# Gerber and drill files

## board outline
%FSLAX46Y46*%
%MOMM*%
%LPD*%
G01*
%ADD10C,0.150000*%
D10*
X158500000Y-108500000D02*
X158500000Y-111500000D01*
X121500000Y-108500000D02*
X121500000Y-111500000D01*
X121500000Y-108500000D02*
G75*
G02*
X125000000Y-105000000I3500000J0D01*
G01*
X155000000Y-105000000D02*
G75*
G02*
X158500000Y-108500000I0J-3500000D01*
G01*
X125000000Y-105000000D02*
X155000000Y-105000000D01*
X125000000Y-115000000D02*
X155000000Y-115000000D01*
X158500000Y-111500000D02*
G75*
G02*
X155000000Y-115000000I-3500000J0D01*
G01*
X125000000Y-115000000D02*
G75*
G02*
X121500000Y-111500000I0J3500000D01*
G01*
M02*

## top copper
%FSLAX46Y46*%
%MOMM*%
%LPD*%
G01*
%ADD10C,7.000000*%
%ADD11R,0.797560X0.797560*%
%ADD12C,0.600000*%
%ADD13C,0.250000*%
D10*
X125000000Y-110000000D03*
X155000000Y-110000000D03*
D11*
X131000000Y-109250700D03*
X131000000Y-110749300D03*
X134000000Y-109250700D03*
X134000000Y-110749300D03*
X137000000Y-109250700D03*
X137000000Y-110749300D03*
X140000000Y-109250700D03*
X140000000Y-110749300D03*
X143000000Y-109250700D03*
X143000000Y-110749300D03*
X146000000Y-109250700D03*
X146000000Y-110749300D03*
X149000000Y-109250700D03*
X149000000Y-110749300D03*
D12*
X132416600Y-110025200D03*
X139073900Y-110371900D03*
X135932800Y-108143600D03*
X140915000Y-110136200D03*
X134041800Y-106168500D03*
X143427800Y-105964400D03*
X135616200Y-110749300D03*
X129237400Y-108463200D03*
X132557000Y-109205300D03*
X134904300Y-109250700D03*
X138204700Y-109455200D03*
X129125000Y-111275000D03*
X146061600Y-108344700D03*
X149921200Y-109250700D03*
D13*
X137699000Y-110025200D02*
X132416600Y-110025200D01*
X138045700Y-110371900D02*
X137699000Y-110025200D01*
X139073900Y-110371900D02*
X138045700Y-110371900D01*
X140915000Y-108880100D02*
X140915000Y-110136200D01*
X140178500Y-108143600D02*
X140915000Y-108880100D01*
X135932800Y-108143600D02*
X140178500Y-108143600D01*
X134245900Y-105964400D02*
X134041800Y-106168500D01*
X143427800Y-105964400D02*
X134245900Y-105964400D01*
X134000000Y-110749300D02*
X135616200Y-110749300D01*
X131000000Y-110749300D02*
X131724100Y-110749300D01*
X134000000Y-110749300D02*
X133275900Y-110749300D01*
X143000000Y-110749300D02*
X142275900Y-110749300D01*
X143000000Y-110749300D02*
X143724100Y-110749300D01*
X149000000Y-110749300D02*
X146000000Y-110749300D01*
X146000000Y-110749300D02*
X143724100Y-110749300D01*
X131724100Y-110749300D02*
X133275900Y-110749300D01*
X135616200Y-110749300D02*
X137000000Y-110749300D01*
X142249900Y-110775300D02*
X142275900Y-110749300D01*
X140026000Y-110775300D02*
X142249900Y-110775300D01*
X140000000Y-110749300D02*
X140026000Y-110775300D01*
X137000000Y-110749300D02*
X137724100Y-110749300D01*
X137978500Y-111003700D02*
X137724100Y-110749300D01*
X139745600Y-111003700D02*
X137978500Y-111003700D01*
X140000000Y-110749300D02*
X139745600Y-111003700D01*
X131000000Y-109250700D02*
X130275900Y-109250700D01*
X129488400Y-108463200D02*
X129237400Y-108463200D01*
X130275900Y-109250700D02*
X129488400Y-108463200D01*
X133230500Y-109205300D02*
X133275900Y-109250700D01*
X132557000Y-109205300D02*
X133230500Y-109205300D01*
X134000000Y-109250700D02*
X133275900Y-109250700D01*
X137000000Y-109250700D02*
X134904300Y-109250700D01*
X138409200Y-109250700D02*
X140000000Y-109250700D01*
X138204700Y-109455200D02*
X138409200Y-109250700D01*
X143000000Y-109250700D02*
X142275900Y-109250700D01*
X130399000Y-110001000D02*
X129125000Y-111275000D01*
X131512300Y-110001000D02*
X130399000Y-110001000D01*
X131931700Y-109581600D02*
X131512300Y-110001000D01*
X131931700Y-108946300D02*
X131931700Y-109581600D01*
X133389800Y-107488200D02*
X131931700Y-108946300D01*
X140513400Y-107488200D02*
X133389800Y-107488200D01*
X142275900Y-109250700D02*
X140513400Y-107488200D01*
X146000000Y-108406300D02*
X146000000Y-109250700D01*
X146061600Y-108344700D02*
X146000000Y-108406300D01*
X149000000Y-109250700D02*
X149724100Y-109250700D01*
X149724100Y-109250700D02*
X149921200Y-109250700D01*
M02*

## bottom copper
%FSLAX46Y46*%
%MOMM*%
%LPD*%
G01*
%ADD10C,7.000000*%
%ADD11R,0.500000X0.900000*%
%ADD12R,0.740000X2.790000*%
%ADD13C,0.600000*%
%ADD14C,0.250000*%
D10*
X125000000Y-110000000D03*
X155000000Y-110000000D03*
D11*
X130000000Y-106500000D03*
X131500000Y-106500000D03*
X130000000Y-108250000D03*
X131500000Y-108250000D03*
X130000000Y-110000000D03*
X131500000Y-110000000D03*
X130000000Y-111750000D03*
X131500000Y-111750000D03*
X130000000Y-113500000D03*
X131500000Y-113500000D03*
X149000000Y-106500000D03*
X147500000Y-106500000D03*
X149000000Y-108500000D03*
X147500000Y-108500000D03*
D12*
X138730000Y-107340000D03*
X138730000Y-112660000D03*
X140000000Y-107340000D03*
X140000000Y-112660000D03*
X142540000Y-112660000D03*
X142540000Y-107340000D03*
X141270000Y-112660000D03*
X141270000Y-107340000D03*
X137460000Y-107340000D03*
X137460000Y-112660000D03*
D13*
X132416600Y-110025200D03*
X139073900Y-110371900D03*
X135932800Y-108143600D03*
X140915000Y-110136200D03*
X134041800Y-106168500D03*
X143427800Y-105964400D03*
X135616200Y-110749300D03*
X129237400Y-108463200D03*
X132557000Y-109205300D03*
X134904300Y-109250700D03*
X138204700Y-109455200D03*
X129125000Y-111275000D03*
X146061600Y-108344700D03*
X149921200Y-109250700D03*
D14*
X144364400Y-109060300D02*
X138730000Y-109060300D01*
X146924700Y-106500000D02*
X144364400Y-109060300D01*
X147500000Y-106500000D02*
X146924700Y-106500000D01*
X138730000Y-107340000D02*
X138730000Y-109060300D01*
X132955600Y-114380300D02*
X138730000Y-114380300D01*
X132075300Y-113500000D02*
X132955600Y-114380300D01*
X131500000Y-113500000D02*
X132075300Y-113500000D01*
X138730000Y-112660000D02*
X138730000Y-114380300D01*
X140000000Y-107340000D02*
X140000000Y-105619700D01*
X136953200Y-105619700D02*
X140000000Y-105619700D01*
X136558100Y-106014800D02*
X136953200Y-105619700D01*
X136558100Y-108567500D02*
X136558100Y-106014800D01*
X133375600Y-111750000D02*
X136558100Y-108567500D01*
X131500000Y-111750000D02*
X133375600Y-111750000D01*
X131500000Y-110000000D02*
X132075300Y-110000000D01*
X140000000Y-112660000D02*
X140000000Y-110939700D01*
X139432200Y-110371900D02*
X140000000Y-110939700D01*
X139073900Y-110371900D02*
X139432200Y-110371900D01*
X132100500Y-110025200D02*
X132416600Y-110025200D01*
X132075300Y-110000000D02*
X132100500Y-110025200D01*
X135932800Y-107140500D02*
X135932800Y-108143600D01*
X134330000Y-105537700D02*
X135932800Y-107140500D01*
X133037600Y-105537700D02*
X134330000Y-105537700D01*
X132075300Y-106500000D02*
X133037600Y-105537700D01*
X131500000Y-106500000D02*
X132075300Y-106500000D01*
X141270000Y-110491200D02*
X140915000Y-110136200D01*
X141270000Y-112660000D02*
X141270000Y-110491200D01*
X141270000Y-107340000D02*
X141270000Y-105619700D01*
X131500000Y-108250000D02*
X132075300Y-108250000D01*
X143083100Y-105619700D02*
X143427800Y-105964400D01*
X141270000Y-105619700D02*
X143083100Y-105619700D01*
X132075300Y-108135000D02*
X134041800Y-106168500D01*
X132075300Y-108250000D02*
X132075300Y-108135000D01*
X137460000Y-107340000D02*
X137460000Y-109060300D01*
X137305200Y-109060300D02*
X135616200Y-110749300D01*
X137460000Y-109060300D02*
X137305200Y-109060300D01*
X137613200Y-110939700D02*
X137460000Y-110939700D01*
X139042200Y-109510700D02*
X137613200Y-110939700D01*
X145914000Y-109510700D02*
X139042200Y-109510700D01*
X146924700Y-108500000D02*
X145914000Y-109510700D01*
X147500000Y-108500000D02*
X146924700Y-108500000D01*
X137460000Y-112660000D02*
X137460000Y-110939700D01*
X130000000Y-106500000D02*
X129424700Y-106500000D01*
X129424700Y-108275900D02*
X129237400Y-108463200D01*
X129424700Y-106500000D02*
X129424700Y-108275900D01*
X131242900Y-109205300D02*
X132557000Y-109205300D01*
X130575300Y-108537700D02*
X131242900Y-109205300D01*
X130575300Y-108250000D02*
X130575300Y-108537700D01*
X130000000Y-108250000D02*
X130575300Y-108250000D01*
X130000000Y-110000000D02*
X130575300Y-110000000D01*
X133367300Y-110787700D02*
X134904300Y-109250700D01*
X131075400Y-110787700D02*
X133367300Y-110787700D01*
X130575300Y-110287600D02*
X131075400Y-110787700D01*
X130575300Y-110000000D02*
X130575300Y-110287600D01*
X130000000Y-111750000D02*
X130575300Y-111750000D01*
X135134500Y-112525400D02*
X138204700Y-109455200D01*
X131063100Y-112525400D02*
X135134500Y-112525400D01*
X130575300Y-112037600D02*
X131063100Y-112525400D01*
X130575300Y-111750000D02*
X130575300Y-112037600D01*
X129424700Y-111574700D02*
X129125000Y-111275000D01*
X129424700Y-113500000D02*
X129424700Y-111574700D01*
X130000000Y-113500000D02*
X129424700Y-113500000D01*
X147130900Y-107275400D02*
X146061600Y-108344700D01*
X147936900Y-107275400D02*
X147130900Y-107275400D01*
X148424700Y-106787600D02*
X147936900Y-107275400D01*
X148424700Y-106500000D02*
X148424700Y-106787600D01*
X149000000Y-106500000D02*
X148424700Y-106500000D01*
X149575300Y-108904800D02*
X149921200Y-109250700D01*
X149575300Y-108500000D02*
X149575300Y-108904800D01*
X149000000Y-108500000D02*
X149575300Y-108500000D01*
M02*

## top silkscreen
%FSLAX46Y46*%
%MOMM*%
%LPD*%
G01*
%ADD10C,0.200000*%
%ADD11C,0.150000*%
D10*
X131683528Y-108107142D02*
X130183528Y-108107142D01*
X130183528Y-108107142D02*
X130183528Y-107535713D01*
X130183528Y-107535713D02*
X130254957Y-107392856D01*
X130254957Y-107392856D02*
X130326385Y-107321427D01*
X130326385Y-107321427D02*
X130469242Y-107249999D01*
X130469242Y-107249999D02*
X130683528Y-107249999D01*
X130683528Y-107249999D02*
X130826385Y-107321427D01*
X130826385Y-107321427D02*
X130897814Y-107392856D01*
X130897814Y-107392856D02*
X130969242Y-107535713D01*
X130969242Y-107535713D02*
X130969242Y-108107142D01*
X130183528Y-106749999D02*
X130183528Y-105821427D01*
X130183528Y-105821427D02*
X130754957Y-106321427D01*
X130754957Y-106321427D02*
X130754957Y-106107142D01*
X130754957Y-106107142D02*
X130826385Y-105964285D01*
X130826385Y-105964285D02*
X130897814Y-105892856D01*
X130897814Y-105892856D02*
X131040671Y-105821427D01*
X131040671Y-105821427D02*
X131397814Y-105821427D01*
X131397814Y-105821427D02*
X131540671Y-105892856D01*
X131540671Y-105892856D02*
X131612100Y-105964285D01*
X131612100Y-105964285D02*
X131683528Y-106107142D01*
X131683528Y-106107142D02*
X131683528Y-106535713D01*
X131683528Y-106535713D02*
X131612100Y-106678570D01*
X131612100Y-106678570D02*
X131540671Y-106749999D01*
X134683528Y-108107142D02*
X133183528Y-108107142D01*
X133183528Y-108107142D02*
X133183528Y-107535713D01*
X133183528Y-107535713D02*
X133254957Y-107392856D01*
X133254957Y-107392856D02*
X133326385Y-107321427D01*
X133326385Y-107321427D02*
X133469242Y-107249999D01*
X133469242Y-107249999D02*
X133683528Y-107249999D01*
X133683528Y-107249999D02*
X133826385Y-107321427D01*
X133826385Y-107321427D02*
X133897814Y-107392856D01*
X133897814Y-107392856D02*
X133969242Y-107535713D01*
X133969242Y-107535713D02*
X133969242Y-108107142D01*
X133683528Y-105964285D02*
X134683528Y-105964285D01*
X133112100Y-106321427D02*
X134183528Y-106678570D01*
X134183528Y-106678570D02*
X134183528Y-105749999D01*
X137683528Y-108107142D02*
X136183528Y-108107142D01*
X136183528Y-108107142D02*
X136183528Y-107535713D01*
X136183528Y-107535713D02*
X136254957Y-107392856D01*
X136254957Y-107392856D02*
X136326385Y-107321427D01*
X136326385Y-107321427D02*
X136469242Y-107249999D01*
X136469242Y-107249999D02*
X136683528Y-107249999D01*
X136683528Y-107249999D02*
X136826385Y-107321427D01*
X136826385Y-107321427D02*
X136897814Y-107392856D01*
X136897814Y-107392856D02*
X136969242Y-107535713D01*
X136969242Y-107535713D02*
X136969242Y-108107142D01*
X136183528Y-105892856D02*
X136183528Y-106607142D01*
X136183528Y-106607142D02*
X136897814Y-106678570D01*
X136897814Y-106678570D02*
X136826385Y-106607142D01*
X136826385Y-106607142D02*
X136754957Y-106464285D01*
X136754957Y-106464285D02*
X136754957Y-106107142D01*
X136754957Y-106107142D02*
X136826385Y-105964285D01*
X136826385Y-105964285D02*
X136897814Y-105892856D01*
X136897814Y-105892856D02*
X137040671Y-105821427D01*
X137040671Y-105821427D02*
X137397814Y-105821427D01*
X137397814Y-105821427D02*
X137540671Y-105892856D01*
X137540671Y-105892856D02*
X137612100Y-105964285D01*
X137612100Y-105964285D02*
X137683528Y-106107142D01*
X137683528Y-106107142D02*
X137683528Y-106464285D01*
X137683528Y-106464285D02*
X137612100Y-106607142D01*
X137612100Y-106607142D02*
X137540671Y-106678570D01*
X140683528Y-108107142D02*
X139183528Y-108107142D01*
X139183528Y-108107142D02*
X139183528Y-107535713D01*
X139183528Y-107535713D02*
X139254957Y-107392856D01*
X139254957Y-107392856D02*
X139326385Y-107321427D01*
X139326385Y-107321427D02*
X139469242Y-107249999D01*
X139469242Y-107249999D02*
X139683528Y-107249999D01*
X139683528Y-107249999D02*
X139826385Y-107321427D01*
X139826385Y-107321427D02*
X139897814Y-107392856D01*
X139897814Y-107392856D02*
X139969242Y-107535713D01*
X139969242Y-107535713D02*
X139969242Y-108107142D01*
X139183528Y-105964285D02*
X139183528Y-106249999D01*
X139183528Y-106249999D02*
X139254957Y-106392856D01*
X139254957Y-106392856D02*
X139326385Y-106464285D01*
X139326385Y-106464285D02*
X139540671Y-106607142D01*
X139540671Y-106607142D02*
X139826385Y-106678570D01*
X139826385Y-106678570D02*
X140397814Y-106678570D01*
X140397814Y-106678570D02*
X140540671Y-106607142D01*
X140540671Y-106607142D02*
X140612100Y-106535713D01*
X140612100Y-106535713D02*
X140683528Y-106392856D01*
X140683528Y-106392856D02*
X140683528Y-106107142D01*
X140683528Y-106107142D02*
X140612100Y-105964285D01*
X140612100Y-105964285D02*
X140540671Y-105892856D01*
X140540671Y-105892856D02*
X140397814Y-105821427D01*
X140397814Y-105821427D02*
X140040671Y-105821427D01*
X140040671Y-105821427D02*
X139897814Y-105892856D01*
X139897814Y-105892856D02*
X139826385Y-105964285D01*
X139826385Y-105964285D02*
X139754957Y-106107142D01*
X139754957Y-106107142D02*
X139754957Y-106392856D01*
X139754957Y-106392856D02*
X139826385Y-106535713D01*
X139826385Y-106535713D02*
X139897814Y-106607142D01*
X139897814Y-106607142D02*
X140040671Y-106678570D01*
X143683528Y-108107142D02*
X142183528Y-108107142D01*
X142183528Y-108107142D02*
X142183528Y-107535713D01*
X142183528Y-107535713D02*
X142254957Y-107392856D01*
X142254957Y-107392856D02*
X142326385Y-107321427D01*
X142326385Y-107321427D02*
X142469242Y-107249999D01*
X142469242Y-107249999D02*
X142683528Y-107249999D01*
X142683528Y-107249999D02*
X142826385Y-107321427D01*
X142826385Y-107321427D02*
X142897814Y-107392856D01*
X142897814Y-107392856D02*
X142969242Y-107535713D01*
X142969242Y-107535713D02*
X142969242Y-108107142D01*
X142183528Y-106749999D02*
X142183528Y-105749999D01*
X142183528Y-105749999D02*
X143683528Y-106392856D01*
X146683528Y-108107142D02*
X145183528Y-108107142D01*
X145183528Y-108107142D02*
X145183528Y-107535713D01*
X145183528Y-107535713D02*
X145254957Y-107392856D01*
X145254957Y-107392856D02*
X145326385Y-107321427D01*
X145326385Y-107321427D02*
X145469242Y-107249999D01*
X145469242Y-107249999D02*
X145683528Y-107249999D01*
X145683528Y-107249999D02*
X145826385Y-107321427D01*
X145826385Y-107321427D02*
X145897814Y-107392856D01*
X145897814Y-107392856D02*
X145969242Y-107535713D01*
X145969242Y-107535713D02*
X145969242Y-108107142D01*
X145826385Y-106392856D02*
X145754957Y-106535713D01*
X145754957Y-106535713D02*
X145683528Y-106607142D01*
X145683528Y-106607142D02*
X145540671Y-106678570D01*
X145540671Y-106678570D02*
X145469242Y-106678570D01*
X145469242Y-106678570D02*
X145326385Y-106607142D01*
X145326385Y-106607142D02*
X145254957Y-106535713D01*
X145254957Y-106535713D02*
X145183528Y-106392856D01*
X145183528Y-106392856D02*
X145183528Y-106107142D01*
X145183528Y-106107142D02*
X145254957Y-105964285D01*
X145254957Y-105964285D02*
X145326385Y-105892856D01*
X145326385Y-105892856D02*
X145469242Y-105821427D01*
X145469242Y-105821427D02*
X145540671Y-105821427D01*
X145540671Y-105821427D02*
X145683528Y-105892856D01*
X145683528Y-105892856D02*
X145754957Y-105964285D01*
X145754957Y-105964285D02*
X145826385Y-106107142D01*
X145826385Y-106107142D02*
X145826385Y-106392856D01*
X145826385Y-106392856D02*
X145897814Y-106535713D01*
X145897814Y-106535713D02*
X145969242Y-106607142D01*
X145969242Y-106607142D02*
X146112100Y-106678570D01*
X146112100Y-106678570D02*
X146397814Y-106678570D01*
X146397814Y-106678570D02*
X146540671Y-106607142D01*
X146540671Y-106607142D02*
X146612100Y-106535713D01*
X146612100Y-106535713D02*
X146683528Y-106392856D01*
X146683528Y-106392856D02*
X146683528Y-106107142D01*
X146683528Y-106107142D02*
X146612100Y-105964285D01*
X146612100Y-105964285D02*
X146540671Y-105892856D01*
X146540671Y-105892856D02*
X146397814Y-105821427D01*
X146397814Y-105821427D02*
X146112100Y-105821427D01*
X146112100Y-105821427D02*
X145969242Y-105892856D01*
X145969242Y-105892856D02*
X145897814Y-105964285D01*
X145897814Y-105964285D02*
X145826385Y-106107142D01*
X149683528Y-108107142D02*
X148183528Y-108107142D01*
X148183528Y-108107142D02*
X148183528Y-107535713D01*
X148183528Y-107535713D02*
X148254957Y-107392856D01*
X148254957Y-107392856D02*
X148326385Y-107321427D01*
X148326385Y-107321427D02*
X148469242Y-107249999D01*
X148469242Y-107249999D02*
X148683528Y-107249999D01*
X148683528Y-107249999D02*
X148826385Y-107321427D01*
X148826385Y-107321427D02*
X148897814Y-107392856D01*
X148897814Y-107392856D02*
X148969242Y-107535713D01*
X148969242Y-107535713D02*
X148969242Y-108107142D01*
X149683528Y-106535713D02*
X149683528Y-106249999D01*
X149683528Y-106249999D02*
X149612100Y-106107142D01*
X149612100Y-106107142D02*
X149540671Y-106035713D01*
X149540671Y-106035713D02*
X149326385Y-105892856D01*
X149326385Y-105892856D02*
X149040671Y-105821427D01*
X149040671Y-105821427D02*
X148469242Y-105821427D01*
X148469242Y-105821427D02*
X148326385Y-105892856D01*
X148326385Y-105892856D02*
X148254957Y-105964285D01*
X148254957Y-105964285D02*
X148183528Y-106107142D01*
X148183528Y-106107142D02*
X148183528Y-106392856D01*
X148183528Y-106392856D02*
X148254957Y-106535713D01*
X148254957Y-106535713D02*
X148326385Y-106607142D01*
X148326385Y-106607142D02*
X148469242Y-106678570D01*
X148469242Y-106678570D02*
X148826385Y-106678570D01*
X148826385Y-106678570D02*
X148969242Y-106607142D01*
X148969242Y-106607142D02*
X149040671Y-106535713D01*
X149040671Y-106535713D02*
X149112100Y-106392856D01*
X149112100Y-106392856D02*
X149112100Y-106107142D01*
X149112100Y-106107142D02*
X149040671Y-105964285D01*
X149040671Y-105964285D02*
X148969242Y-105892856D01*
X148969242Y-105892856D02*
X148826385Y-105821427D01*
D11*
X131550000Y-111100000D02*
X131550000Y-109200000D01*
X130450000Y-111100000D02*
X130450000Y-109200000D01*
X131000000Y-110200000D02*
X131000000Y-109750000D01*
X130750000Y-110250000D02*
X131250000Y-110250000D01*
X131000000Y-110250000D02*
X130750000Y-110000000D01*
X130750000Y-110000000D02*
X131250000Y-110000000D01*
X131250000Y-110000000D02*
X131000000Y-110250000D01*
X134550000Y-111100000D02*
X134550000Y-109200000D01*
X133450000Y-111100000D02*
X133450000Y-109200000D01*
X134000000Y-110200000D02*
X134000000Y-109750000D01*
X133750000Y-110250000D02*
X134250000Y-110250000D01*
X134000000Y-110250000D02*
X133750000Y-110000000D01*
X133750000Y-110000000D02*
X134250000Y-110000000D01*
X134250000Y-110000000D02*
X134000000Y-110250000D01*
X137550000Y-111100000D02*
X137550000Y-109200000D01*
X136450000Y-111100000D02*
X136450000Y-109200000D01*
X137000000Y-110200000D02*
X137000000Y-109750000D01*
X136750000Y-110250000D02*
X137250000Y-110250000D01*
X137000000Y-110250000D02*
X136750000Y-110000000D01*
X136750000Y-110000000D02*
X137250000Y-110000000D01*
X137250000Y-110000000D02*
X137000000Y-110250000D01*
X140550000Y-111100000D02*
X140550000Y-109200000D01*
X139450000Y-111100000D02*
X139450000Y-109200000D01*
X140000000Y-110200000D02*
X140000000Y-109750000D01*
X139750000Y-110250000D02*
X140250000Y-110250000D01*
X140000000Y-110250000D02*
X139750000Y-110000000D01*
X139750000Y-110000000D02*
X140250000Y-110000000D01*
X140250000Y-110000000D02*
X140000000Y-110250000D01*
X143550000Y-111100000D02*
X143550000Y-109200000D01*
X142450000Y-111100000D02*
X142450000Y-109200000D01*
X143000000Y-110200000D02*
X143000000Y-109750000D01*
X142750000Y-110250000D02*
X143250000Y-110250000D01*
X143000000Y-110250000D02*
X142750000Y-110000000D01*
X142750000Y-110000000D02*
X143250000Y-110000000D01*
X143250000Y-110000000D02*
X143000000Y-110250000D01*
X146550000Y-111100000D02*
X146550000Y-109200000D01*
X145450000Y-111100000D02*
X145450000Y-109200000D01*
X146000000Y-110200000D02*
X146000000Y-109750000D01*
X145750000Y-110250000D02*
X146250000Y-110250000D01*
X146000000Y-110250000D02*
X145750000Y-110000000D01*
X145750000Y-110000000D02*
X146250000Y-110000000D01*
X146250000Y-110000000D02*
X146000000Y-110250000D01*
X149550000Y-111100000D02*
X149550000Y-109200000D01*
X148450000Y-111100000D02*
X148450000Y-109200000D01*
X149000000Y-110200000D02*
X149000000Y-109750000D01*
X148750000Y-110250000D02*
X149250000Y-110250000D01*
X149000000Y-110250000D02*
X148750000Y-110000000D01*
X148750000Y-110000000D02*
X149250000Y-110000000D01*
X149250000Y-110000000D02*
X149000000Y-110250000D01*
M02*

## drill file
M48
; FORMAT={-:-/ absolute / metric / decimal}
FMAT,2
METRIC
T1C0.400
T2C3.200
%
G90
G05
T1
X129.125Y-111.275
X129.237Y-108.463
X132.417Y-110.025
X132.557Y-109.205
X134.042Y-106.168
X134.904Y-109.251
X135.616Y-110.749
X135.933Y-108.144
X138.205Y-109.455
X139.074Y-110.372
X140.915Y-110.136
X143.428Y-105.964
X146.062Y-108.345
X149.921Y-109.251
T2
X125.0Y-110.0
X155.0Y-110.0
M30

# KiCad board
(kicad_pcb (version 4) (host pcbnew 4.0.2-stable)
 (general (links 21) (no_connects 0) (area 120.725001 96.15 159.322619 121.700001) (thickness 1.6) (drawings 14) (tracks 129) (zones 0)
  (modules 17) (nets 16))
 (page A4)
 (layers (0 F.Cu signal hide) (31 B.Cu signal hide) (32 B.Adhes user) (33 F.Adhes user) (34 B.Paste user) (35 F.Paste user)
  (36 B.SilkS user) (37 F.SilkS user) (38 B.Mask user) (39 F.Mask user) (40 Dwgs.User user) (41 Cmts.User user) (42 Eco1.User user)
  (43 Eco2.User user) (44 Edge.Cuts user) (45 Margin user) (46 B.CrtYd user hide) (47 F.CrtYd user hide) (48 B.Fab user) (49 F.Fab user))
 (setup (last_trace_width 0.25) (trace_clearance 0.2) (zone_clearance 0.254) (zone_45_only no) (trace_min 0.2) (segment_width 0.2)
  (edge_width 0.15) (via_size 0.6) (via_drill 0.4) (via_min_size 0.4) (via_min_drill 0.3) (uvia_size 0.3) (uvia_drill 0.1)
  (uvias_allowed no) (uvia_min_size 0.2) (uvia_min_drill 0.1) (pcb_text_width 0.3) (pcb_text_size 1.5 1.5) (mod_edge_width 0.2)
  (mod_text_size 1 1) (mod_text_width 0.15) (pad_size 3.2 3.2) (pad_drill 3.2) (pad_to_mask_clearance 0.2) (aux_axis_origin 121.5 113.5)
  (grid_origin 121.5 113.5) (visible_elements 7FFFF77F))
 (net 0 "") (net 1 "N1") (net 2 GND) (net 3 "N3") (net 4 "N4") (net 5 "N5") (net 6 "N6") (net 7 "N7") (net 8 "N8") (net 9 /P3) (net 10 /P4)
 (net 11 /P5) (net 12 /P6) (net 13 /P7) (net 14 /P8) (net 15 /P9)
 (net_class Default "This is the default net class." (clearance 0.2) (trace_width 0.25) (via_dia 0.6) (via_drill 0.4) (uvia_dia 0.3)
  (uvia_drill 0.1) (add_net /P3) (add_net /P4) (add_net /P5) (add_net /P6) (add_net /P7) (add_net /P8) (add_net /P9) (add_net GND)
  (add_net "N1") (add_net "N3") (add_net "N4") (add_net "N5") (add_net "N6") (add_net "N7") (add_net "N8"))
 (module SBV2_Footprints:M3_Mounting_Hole (layer F.Cu) (at 125 110)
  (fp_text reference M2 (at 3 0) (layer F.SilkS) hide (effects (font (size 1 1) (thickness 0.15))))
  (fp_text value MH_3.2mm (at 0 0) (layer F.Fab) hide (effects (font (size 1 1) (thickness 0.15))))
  (pad "" np_thru_hole circle (at 0 0) (size 7 7) (drill 3.2) (layers *.Cu *.Mask)))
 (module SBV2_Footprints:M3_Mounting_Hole (layer F.Cu) (at 155 110)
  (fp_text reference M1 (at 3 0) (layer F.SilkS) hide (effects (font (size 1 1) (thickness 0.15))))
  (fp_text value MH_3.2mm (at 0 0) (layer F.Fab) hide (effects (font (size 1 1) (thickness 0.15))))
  (pad "" np_thru_hole circle (at 0 0) (size 7 7) (drill 3.2) (layers *.Cu *.Mask)))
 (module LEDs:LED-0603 (layer F.Cu) (at 131 110 90)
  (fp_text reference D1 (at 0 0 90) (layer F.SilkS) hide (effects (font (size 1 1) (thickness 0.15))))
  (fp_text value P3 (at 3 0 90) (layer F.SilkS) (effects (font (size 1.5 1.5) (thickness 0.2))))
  (fp_line (start -1.1 0.55) (end 0.8 0.55) (layer F.SilkS) (width 0.15))
  (fp_line (start -1.1 -0.55) (end 0.8 -0.55) (layer F.SilkS) (width 0.15))
  (fp_line (start -0.2 0) (end 0.25 0) (layer F.SilkS) (width 0.15))
  (fp_line (start -0.25 -0.25) (end -0.25 0.25) (layer F.SilkS) (width 0.15))
  (fp_line (start -0.25 0) (end 0 -0.25) (layer F.SilkS) (width 0.15))
  (fp_line (start 0 -0.25) (end 0 0.25) (layer F.SilkS) (width 0.15))
  (fp_line (start 0 0.25) (end -0.25 0) (layer F.SilkS) (width 0.15))
  (pad 2 smd rect (at 0.7493 0 270) (size 0.79756 0.79756) (layers F.Cu F.Paste F.Mask) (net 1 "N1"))
  (pad 1 smd rect (at -0.7493 0 270) (size 0.79756 0.79756) (layers F.Cu F.Paste F.Mask) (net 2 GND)))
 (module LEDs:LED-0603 (layer F.Cu) (at 134 110 90)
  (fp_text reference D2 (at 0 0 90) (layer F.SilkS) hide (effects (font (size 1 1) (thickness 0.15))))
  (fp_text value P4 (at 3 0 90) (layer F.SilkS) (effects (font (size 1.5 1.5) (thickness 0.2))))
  (fp_line (start -1.1 0.55) (end 0.8 0.55) (layer F.SilkS) (width 0.15))
  (fp_line (start -1.1 -0.55) (end 0.8 -0.55) (layer F.SilkS) (width 0.15))
  (fp_line (start -0.2 0) (end 0.25 0) (layer F.SilkS) (width 0.15))
  (fp_line (start -0.25 -0.25) (end -0.25 0.25) (layer F.SilkS) (width 0.15))
  (fp_line (start -0.25 0) (end 0 -0.25) (layer F.SilkS) (width 0.15))
  (fp_line (start 0 -0.25) (end 0 0.25) (layer F.SilkS) (width 0.15))
  (fp_line (start 0 0.25) (end -0.25 0) (layer F.SilkS) (width 0.15))
  (pad 2 smd rect (at 0.7493 0 270) (size 0.79756 0.79756) (layers F.Cu F.Paste F.Mask) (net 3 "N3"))
  (pad 1 smd rect (at -0.7493 0 270) (size 0.79756 0.79756) (layers F.Cu F.Paste F.Mask) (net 2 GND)))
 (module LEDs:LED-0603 (layer F.Cu) (at 137 110 90)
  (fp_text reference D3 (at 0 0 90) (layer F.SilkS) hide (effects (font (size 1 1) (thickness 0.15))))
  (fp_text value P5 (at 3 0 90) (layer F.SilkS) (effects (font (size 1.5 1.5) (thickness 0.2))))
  (fp_line (start -1.1 0.55) (end 0.8 0.55) (layer F.SilkS) (width 0.15))
  (fp_line (start -1.1 -0.55) (end 0.8 -0.55) (layer F.SilkS) (width 0.15))
  (fp_line (start -0.2 0) (end 0.25 0) (layer F.SilkS) (width 0.15))
  (fp_line (start -0.25 -0.25) (end -0.25 0.25) (layer F.SilkS) (width 0.15))
  (fp_line (start -0.25 0) (end 0 -0.25) (layer F.SilkS) (width 0.15))
  (fp_line (start 0 -0.25) (end 0 0.25) (layer F.SilkS) (width 0.15))
  (fp_line (start 0 0.25) (end -0.25 0) (layer F.SilkS) (width 0.15))
  (pad 2 smd rect (at 0.7493 0 270) (size 0.79756 0.79756) (layers F.Cu F.Paste F.Mask) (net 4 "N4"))
  (pad 1 smd rect (at -0.7493 0 270) (size 0.79756 0.79756) (layers F.Cu F.Paste F.Mask) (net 2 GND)))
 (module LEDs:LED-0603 (layer F.Cu) (at 140 110 90)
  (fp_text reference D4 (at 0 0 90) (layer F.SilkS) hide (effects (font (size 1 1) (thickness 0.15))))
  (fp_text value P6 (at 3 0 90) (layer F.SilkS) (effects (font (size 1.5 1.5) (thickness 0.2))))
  (fp_line (start -1.1 0.55) (end 0.8 0.55) (layer F.SilkS) (width 0.15))
  (fp_line (start -1.1 -0.55) (end 0.8 -0.55) (layer F.SilkS) (width 0.15))
  (fp_line (start -0.2 0) (end 0.25 0) (layer F.SilkS) (width 0.15))
  (fp_line (start -0.25 -0.25) (end -0.25 0.25) (layer F.SilkS) (width 0.15))
  (fp_line (start -0.25 0) (end 0 -0.25) (layer F.SilkS) (width 0.15))
  (fp_line (start 0 -0.25) (end 0 0.25) (layer F.SilkS) (width 0.15))
  (fp_line (start 0 0.25) (end -0.25 0) (layer F.SilkS) (width 0.15))
  (pad 2 smd rect (at 0.7493 0 270) (size 0.79756 0.79756) (layers F.Cu F.Paste F.Mask) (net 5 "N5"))
  (pad 1 smd rect (at -0.7493 0 270) (size 0.79756 0.79756) (layers F.Cu F.Paste F.Mask) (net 2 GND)))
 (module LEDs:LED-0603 (layer F.Cu) (at 143 110 90)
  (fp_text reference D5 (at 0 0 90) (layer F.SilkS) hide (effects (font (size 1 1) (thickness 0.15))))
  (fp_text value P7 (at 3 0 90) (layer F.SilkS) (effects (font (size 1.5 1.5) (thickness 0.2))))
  (fp_line (start -1.1 0.55) (end 0.8 0.55) (layer F.SilkS) (width 0.15))
  (fp_line (start -1.1 -0.55) (end 0.8 -0.55) (layer F.SilkS) (width 0.15))
  (fp_line (start -0.2 0) (end 0.25 0) (layer F.SilkS) (width 0.15))
  (fp_line (start -0.25 -0.25) (end -0.25 0.25) (layer F.SilkS) (width 0.15))
  (fp_line (start -0.25 0) (end 0 -0.25) (layer F.SilkS) (width 0.15))
  (fp_line (start 0 -0.25) (end 0 0.25) (layer F.SilkS) (width 0.15))
  (fp_line (start 0 0.25) (end -0.25 0) (layer F.SilkS) (width 0.15))
  (pad 2 smd rect (at 0.7493 0 270) (size 0.79756 0.79756) (layers F.Cu F.Paste F.Mask) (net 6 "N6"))
  (pad 1 smd rect (at -0.7493 0 270) (size 0.79756 0.79756) (layers F.Cu F.Paste F.Mask) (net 2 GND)))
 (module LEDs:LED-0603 (layer F.Cu) (at 146 110 90)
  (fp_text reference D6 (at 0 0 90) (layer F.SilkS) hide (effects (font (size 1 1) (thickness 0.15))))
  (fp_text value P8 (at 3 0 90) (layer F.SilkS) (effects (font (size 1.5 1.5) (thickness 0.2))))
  (fp_line (start -1.1 0.55) (end 0.8 0.55) (layer F.SilkS) (width 0.15))
  (fp_line (start -1.1 -0.55) (end 0.8 -0.55) (layer F.SilkS) (width 0.15))
  (fp_line (start -0.2 0) (end 0.25 0) (layer F.SilkS) (width 0.15))
  (fp_line (start -0.25 -0.25) (end -0.25 0.25) (layer F.SilkS) (width 0.15))
  (fp_line (start -0.25 0) (end 0 -0.25) (layer F.SilkS) (width 0.15))
  (fp_line (start 0 -0.25) (end 0 0.25) (layer F.SilkS) (width 0.15))
  (fp_line (start 0 0.25) (end -0.25 0) (layer F.SilkS) (width 0.15))
  (pad 2 smd rect (at 0.7493 0 270) (size 0.79756 0.79756) (layers F.Cu F.Paste F.Mask) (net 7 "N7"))
  (pad 1 smd rect (at -0.7493 0 270) (size 0.79756 0.79756) (layers F.Cu F.Paste F.Mask) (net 2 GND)))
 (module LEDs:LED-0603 (layer F.Cu) (at 149 110 90)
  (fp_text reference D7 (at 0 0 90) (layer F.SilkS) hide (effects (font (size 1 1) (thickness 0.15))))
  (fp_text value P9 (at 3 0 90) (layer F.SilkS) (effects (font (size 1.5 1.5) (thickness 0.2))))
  (fp_line (start -1.1 0.55) (end 0.8 0.55) (layer F.SilkS) (width 0.15))
  (fp_line (start -1.1 -0.55) (end 0.8 -0.55) (layer F.SilkS) (width 0.15))
  (fp_line (start -0.2 0) (end 0.25 0) (layer F.SilkS) (width 0.15))
  (fp_line (start -0.25 -0.25) (end -0.25 0.25) (layer F.SilkS) (width 0.15))
  (fp_line (start -0.25 0) (end 0 -0.25) (layer F.SilkS) (width 0.15))
  (fp_line (start 0 -0.25) (end 0 0.25) (layer F.SilkS) (width 0.15))
  (fp_line (start 0 0.25) (end -0.25 0) (layer F.SilkS) (width 0.15))
  (pad 2 smd rect (at 0.7493 0 270) (size 0.79756 0.79756) (layers F.Cu F.Paste F.Mask) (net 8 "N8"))
  (pad 1 smd rect (at -0.7493 0 270) (size 0.79756 0.79756) (layers F.Cu F.Paste F.Mask) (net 2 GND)))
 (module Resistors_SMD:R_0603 (layer B.Cu) (at 130.75 106.5)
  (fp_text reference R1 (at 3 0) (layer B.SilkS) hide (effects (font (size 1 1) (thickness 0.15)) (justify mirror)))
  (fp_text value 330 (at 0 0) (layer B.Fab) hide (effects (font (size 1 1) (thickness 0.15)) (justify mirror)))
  (pad 1 smd rect (at -0.75 0) (size 0.5 0.9) (layers B.Cu B.Paste B.Mask) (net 1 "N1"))
  (pad 2 smd rect (at 0.75 0) (size 0.5 0.9) (layers B.Cu B.Paste B.Mask) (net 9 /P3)))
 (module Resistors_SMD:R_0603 (layer B.Cu) (at 130.75 108.25)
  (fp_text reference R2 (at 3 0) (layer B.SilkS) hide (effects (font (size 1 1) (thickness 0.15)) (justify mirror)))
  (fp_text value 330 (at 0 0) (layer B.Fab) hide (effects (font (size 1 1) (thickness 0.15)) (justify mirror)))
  (pad 1 smd rect (at -0.75 0) (size 0.5 0.9) (layers B.Cu B.Paste B.Mask) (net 3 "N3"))
  (pad 2 smd rect (at 0.75 0) (size 0.5 0.9) (layers B.Cu B.Paste B.Mask) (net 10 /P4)))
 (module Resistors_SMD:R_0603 (layer B.Cu) (at 130.75 110)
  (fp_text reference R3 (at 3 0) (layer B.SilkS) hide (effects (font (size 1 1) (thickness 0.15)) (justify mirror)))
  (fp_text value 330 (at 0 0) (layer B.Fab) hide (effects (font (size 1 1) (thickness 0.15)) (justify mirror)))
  (pad 1 smd rect (at -0.75 0) (size 0.5 0.9) (layers B.Cu B.Paste B.Mask) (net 4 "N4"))
  (pad 2 smd rect (at 0.75 0) (size 0.5 0.9) (layers B.Cu B.Paste B.Mask) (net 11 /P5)))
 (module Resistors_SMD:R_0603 (layer B.Cu) (at 130.75 111.75)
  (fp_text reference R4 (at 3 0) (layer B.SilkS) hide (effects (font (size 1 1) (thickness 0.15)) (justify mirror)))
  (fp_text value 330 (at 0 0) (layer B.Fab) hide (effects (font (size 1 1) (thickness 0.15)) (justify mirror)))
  (pad 1 smd rect (at -0.75 0) (size 0.5 0.9) (layers B.Cu B.Paste B.Mask) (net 5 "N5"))
  (pad 2 smd rect (at 0.75 0) (size 0.5 0.9) (layers B.Cu B.Paste B.Mask) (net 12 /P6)))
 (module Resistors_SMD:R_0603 (layer B.Cu) (at 130.75 113.5)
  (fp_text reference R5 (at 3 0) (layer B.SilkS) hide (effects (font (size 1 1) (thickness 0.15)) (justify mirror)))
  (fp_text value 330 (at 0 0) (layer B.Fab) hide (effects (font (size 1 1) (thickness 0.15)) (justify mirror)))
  (pad 1 smd rect (at -0.75 0) (size 0.5 0.9) (layers B.Cu B.Paste B.Mask) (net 6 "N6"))
  (pad 2 smd rect (at 0.75 0) (size 0.5 0.9) (layers B.Cu B.Paste B.Mask) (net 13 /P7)))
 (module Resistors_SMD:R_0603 (layer B.Cu) (at 148.25 106.5 180)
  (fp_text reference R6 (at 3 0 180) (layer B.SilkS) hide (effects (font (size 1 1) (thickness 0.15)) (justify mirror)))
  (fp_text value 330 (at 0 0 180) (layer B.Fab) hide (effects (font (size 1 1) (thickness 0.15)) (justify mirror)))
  (pad 1 smd rect (at -0.75 0 180) (size 0.5 0.9) (layers B.Cu B.Paste B.Mask) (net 7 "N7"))
  (pad 2 smd rect (at 0.75 0 180) (size 0.5 0.9) (layers B.Cu B.Paste B.Mask) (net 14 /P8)))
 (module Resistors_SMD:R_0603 (layer B.Cu) (at 148.25 108.5 180)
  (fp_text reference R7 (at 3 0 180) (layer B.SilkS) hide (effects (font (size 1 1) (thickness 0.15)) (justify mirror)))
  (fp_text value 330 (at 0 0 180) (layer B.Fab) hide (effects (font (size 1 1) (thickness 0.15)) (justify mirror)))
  (pad 1 smd rect (at -0.75 0 180) (size 0.5 0.9) (layers B.Cu B.Paste B.Mask) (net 8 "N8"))
  (pad 2 smd rect (at 0.75 0 180) (size 0.5 0.9) (layers B.Cu B.Paste B.Mask) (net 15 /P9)))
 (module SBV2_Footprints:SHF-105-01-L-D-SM (layer B.Cu) (at 140 110 180)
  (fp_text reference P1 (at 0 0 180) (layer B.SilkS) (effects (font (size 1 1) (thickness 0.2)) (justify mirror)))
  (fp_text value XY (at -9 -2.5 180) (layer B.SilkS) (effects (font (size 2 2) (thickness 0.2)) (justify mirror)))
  (pad 8 smd rect (at 1.27 2.66 180) (size 0.74 2.79) (layers B.Cu B.Paste B.Mask) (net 14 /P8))
  (pad 7 smd rect (at 1.27 -2.66 180) (size 0.74 2.79) (layers B.Cu B.Paste B.Mask) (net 13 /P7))
  (pad 6 smd rect (at 0 2.66 180) (size 0.74 2.79) (layers B.Cu B.Paste B.Mask) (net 12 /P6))
  (pad 5 smd rect (at 0 -2.66) (size 0.74 2.79) (layers B.Cu B.Paste B.Mask) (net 11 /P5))
  (pad 1 smd rect (at -2.54 -2.66 180) (size 0.74 2.79) (layers B.Cu B.Paste B.Mask))
  (pad 2 smd rect (at -2.54 2.66 180) (size 0.74 2.79) (layers B.Cu B.Paste B.Mask))
  (pad 3 smd rect (at -1.27 -2.66 180) (size 0.74 2.79) (layers B.Cu B.Paste B.Mask) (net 9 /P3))
  (pad 4 smd rect (at -1.27 2.66 180) (size 0.74 2.79) (layers B.Cu B.Paste B.Mask) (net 10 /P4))
  (pad 10 smd rect (at 2.54 2.66 180) (size 0.74 2.79) (layers B.Cu B.Paste B.Mask) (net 2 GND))
  (pad 9 smd rect (at 2.54 -2.66 180) (size 0.74 2.79) (layers B.Cu B.Paste B.Mask) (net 15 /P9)))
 (gr_line (start 158.5 108.5) (end 158.5 111.5) (angle 90) (layer Edge.Cuts) (width 0.15))
 (gr_line (start 121.5 108.5) (end 121.5 111.5) (angle 90) (layer Edge.Cuts) (width 0.15))
 (gr_arc (start 125 108.5) (end 121.5 108.5) (angle 90) (layer Edge.Cuts) (width 0.15))
 (gr_arc (start 155 108.5) (end 155 105) (angle 90) (layer Edge.Cuts) (width 0.15))
 (gr_line (start 125 105) (end 155 105) (angle 90) (layer Edge.Cuts) (width 0.15))
 (gr_line (start 125 115) (end 155 115) (angle 90) (layer Edge.Cuts) (width 0.15))
 (gr_arc (start 155 111.5) (end 158.5 111.5) (angle 90) (layer Edge.Cuts) (width 0.15))
 (gr_arc (start 125 111.5) (end 125 115) (angle 90) (layer Edge.Cuts) (width 0.15))
 (segment (start 144.3644 109.0603) (end 138.73 109.0603) (width 0.25) (layer B.Cu) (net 14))
 (segment (start 146.9247 106.5) (end 144.3644 109.0603) (width 0.25) (layer B.Cu) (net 14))
 (segment (start 147.5 106.5) (end 146.9247 106.5) (width 0.25) (layer B.Cu) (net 14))
 (segment (start 138.73 107.34) (end 138.73 109.0603) (width 0.25) (layer B.Cu) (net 14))
 (segment (start 132.9556 114.3803) (end 138.73 114.3803) (width 0.25) (layer B.Cu) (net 13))
 (segment (start 132.0753 113.5) (end 132.9556 114.3803) (width 0.25) (layer B.Cu) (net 13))
 (segment (start 131.5 113.5) (end 132.0753 113.5) (width 0.25) (layer B.Cu) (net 13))
 (segment (start 138.73 112.66) (end 138.73 114.3803) (width 0.25) (layer B.Cu) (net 13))
 (segment (start 140 107.34) (end 140 105.6197) (width 0.25) (layer B.Cu) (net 12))
 (segment (start 136.9532 105.6197) (end 140 105.6197) (width 0.25) (layer B.Cu) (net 12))
 (segment (start 136.5581 106.0148) (end 136.9532 105.6197) (width 0.25) (layer B.Cu) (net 12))
 (segment (start 136.5581 108.5675) (end 136.5581 106.0148) (width 0.25) (layer B.Cu) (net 12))
 (segment (start 133.3756 111.75) (end 136.5581 108.5675) (width 0.25) (layer B.Cu) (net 12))
 (segment (start 131.5 111.75) (end 133.3756 111.75) (width 0.25) (layer B.Cu) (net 12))
 (via (at 132.4166 110.0252) (size 0.6) (layers F.Cu B.Cu) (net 11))
 (via (at 139.0739 110.3719) (size 0.6) (layers F.Cu B.Cu) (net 11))
 (segment (start 131.5 110) (end 132.0753 110) (width 0.25) (layer B.Cu) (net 11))
 (segment (start 140 112.66) (end 140 110.9397) (width 0.25) (layer B.Cu) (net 11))
 (segment (start 139.4322 110.3719) (end 140 110.9397) (width 0.25) (layer B.Cu) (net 11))
 (segment (start 139.0739 110.3719) (end 139.4322 110.3719) (width 0.25) (layer B.Cu) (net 11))
 (segment (start 132.1005 110.0252) (end 132.4166 110.0252) (width 0.25) (layer B.Cu) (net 11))
 (segment (start 132.0753 110) (end 132.1005 110.0252) (width 0.25) (layer B.Cu) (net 11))
 (segment (start 137.699 110.0252) (end 132.4166 110.0252) (width 0.25) (layer F.Cu) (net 11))
 (segment (start 138.0457 110.3719) (end 137.699 110.0252) (width 0.25) (layer F.Cu) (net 11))
 (segment (start 139.0739 110.3719) (end 138.0457 110.3719) (width 0.25) (layer F.Cu) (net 11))
 (via (at 135.9328 108.1436) (size 0.6) (layers F.Cu B.Cu) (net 9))
 (via (at 140.915 110.1362) (size 0.6) (layers F.Cu B.Cu) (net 9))
 (segment (start 135.9328 107.1405) (end 135.9328 108.1436) (width 0.25) (layer B.Cu) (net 9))
 (segment (start 134.33 105.5377) (end 135.9328 107.1405) (width 0.25) (layer B.Cu) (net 9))
 (segment (start 133.0376 105.5377) (end 134.33 105.5377) (width 0.25) (layer B.Cu) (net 9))
 (segment (start 132.0753 106.5) (end 133.0376 105.5377) (width 0.25) (layer B.Cu) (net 9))
 (segment (start 131.5 106.5) (end 132.0753 106.5) (width 0.25) (layer B.Cu) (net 9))
 (segment (start 141.27 110.4912) (end 140.915 110.1362) (width 0.25) (layer B.Cu) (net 9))
 (segment (start 141.27 112.66) (end 141.27 110.4912) (width 0.25) (layer B.Cu) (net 9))
 (segment (start 140.915 108.8801) (end 140.915 110.1362) (width 0.25) (layer F.Cu) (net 9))
 (segment (start 140.1785 108.1436) (end 140.915 108.8801) (width 0.25) (layer F.Cu) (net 9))
 (segment (start 135.9328 108.1436) (end 140.1785 108.1436) (width 0.25) (layer F.Cu) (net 9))
 (via (at 134.0418 106.1685) (size 0.6) (layers F.Cu B.Cu) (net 10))
 (via (at 143.4278 105.9644) (size 0.6) (layers F.Cu B.Cu) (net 10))
 (segment (start 141.27 107.34) (end 141.27 105.6197) (width 0.25) (layer B.Cu) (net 10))
 (segment (start 131.5 108.25) (end 132.0753 108.25) (width 0.25) (layer B.Cu) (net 10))
 (segment (start 143.0831 105.6197) (end 143.4278 105.9644) (width 0.25) (layer B.Cu) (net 10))
 (segment (start 141.27 105.6197) (end 143.0831 105.6197) (width 0.25) (layer B.Cu) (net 10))
 (segment (start 132.0753 108.135) (end 134.0418 106.1685) (width 0.25) (layer B.Cu) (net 10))
 (segment (start 132.0753 108.25) (end 132.0753 108.135) (width 0.25) (layer B.Cu) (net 10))
 (segment (start 134.2459 105.9644) (end 134.0418 106.1685) (width 0.25) (layer F.Cu) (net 10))
 (segment (start 143.4278 105.9644) (end 134.2459 105.9644) (width 0.25) (layer F.Cu) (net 10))
 (via (at 135.6162 110.7493) (size 0.6) (layers F.Cu B.Cu) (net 2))
 (segment (start 137.46 107.34) (end 137.46 109.0603) (width 0.25) (layer B.Cu) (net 2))
 (segment (start 134 110.7493) (end 135.6162 110.7493) (width 0.25) (layer F.Cu) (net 2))
 (segment (start 137.3052 109.0603) (end 135.6162 110.7493) (width 0.25) (layer B.Cu) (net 2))
 (segment (start 137.46 109.0603) (end 137.3052 109.0603) (width 0.25) (layer B.Cu) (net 2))
 (segment (start 131 110.7493) (end 131.7241 110.7493) (width 0.25) (layer F.Cu) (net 2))
 (segment (start 134 110.7493) (end 133.2759 110.7493) (width 0.25) (layer F.Cu) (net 2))
 (segment (start 143 110.7493) (end 142.2759 110.7493) (width 0.25) (layer F.Cu) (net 2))
 (segment (start 143 110.7493) (end 143.7241 110.7493) (width 0.25) (layer F.Cu) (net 2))
 (segment (start 149 110.7493) (end 146 110.7493) (width 0.25) (layer F.Cu) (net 2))
 (segment (start 146 110.7493) (end 143.7241 110.7493) (width 0.25) (layer F.Cu) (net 2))
 (segment (start 131.7241 110.7493) (end 133.2759 110.7493) (width 0.25) (layer F.Cu) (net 2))
 (segment (start 135.6162 110.7493) (end 137 110.7493) (width 0.25) (layer F.Cu) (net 2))
 (segment (start 142.2499 110.7753) (end 142.2759 110.7493) (width 0.25) (layer F.Cu) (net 2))
 (segment (start 140.026 110.7753) (end 142.2499 110.7753) (width 0.25) (layer F.Cu) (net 2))
 (segment (start 140 110.7493) (end 140.026 110.7753) (width 0.25) (layer F.Cu) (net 2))
 (segment (start 137 110.7493) (end 137.7241 110.7493) (width 0.25) (layer F.Cu) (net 2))
 (segment (start 137.9785 111.0037) (end 137.7241 110.7493) (width 0.25) (layer F.Cu) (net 2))
 (segment (start 139.7456 111.0037) (end 137.9785 111.0037) (width 0.25) (layer F.Cu) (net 2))
 (segment (start 140 110.7493) (end 139.7456 111.0037) (width 0.25) (layer F.Cu) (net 2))
 (segment (start 137.6132 110.9397) (end 137.46 110.9397) (width 0.25) (layer B.Cu) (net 15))
 (segment (start 139.0422 109.5107) (end 137.6132 110.9397) (width 0.25) (layer B.Cu) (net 15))
 (segment (start 145.914 109.5107) (end 139.0422 109.5107) (width 0.25) (layer B.Cu) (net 15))
 (segment (start 146.9247 108.5) (end 145.914 109.5107) (width 0.25) (layer B.Cu) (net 15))
 (segment (start 147.5 108.5) (end 146.9247 108.5) (width 0.25) (layer B.Cu) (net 15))
 (segment (start 137.46 112.66) (end 137.46 110.9397) (width 0.25) (layer B.Cu) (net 15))
 (via (at 129.2374 108.4632) (size 0.6) (layers F.Cu B.Cu) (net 1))
 (segment (start 131 109.2507) (end 130.2759 109.2507) (width 0.25) (layer F.Cu) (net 1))
 (segment (start 130 106.5) (end 129.4247 106.5) (width 0.25) (layer B.Cu) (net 1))
 (segment (start 129.4247 108.2759) (end 129.2374 108.4632) (width 0.25) (layer B.Cu) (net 1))
 (segment (start 129.4247 106.5) (end 129.4247 108.2759) (width 0.25) (layer B.Cu) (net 1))
 (segment (start 129.4884 108.4632) (end 129.2374 108.4632) (width 0.25) (layer F.Cu) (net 1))
 (segment (start 130.2759 109.2507) (end 129.4884 108.4632) (width 0.25) (layer F.Cu) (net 1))
 (via (at 132.557 109.2053) (size 0.6) (layers F.Cu B.Cu) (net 3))
 (segment (start 131.2429 109.2053) (end 132.557 109.2053) (width 0.25) (layer B.Cu) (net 3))
 (segment (start 130.5753 108.5377) (end 131.2429 109.2053) (width 0.25) (layer B.Cu) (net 3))
 (segment (start 130.5753 108.25) (end 130.5753 108.5377) (width 0.25) (layer B.Cu) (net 3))
 (segment (start 133.2305 109.2053) (end 133.2759 109.2507) (width 0.25) (layer F.Cu) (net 3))
 (segment (start 132.557 109.2053) (end 133.2305 109.2053) (width 0.25) (layer F.Cu) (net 3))
 (segment (start 134 109.2507) (end 133.2759 109.2507) (width 0.25) (layer F.Cu) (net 3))
 (segment (start 130 108.25) (end 130.5753 108.25) (width 0.25) (layer B.Cu) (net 3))
 (via (at 134.9043 109.2507) (size 0.6) (layers F.Cu B.Cu) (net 4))
 (segment (start 137 109.2507) (end 134.9043 109.2507) (width 0.25) (layer F.Cu) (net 4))
 (segment (start 130 110) (end 130.5753 110) (width 0.25) (layer B.Cu) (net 4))
 (segment (start 133.3673 110.7877) (end 134.9043 109.2507) (width 0.25) (layer B.Cu) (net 4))
 (segment (start 131.0754 110.7877) (end 133.3673 110.7877) (width 0.25) (layer B.Cu) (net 4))
 (segment (start 130.5753 110.2876) (end 131.0754 110.7877) (width 0.25) (layer B.Cu) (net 4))
 (segment (start 130.5753 110) (end 130.5753 110.2876) (width 0.25) (layer B.Cu) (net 4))
 (via (at 138.2047 109.4552) (size 0.6) (layers F.Cu B.Cu) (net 5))
 (segment (start 130 111.75) (end 130.5753 111.75) (width 0.25) (layer B.Cu) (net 5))
 (segment (start 135.1345 112.5254) (end 138.2047 109.4552) (width 0.25) (layer B.Cu) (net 5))
 (segment (start 131.0631 112.5254) (end 135.1345 112.5254) (width 0.25) (layer B.Cu) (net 5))
 (segment (start 130.5753 112.0376) (end 131.0631 112.5254) (width 0.25) (layer B.Cu) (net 5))
 (segment (start 130.5753 111.75) (end 130.5753 112.0376) (width 0.25) (layer B.Cu) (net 5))
 (segment (start 138.4092 109.2507) (end 140 109.2507) (width 0.25) (layer F.Cu) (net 5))
 (segment (start 138.2047 109.4552) (end 138.4092 109.2507) (width 0.25) (layer F.Cu) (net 5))
 (via (at 129.125 111.275) (size 0.6) (layers F.Cu B.Cu) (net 6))
 (segment (start 129.4247 111.5747) (end 129.125 111.275) (width 0.25) (layer B.Cu) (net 6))
 (segment (start 129.4247 113.5) (end 129.4247 111.5747) (width 0.25) (layer B.Cu) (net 6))
 (segment (start 143 109.2507) (end 142.2759 109.2507) (width 0.25) (layer F.Cu) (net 6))
 (segment (start 130 113.5) (end 129.4247 113.5) (width 0.25) (layer B.Cu) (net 6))
 (segment (start 130.399 110.001) (end 129.125 111.275) (width 0.25) (layer F.Cu) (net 6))
 (segment (start 131.5123 110.001) (end 130.399 110.001) (width 0.25) (layer F.Cu) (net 6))
 (segment (start 131.9317 109.5816) (end 131.5123 110.001) (width 0.25) (layer F.Cu) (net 6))
 (segment (start 131.9317 108.9463) (end 131.9317 109.5816) (width 0.25) (layer F.Cu) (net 6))
 (segment (start 133.3898 107.4882) (end 131.9317 108.9463) (width 0.25) (layer F.Cu) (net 6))
 (segment (start 140.5134 107.4882) (end 133.3898 107.4882) (width 0.25) (layer F.Cu) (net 6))
 (segment (start 142.2759 109.2507) (end 140.5134 107.4882) (width 0.25) (layer F.Cu) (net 6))
 (via (at 146.0616 108.3447) (size 0.6) (layers F.Cu B.Cu) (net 7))
 (segment (start 147.1309 107.2754) (end 146.0616 108.3447) (width 0.25) (layer B.Cu) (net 7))
 (segment (start 147.9369 107.2754) (end 147.1309 107.2754) (width 0.25) (layer B.Cu) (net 7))
 (segment (start 148.4247 106.7876) (end 147.9369 107.2754) (width 0.25) (layer B.Cu) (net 7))
 (segment (start 148.4247 106.5) (end 148.4247 106.7876) (width 0.25) (layer B.Cu) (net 7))
 (segment (start 146 108.4063) (end 146 109.2507) (width 0.25) (layer F.Cu) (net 7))
 (segment (start 146.0616 108.3447) (end 146 108.4063) (width 0.25) (layer F.Cu) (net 7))
 (segment (start 149 106.5) (end 148.4247 106.5) (width 0.25) (layer B.Cu) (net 7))
 (via (at 149.9212 109.2507) (size 0.6) (layers F.Cu B.Cu) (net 8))
 (segment (start 149 109.2507) (end 149.7241 109.2507) (width 0.25) (layer F.Cu) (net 8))
 (segment (start 149.5753 108.9048) (end 149.9212 109.2507) (width 0.25) (layer B.Cu) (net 8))
 (segment (start 149.5753 108.5) (end 149.5753 108.9048) (width 0.25) (layer B.Cu) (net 8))
 (segment (start 149.7241 109.2507) (end 149.9212 109.2507) (width 0.25) (layer F.Cu) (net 8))
 (segment (start 149 108.5) (end 149.5753 108.5) (width 0.25) (layer B.Cu) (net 8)))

